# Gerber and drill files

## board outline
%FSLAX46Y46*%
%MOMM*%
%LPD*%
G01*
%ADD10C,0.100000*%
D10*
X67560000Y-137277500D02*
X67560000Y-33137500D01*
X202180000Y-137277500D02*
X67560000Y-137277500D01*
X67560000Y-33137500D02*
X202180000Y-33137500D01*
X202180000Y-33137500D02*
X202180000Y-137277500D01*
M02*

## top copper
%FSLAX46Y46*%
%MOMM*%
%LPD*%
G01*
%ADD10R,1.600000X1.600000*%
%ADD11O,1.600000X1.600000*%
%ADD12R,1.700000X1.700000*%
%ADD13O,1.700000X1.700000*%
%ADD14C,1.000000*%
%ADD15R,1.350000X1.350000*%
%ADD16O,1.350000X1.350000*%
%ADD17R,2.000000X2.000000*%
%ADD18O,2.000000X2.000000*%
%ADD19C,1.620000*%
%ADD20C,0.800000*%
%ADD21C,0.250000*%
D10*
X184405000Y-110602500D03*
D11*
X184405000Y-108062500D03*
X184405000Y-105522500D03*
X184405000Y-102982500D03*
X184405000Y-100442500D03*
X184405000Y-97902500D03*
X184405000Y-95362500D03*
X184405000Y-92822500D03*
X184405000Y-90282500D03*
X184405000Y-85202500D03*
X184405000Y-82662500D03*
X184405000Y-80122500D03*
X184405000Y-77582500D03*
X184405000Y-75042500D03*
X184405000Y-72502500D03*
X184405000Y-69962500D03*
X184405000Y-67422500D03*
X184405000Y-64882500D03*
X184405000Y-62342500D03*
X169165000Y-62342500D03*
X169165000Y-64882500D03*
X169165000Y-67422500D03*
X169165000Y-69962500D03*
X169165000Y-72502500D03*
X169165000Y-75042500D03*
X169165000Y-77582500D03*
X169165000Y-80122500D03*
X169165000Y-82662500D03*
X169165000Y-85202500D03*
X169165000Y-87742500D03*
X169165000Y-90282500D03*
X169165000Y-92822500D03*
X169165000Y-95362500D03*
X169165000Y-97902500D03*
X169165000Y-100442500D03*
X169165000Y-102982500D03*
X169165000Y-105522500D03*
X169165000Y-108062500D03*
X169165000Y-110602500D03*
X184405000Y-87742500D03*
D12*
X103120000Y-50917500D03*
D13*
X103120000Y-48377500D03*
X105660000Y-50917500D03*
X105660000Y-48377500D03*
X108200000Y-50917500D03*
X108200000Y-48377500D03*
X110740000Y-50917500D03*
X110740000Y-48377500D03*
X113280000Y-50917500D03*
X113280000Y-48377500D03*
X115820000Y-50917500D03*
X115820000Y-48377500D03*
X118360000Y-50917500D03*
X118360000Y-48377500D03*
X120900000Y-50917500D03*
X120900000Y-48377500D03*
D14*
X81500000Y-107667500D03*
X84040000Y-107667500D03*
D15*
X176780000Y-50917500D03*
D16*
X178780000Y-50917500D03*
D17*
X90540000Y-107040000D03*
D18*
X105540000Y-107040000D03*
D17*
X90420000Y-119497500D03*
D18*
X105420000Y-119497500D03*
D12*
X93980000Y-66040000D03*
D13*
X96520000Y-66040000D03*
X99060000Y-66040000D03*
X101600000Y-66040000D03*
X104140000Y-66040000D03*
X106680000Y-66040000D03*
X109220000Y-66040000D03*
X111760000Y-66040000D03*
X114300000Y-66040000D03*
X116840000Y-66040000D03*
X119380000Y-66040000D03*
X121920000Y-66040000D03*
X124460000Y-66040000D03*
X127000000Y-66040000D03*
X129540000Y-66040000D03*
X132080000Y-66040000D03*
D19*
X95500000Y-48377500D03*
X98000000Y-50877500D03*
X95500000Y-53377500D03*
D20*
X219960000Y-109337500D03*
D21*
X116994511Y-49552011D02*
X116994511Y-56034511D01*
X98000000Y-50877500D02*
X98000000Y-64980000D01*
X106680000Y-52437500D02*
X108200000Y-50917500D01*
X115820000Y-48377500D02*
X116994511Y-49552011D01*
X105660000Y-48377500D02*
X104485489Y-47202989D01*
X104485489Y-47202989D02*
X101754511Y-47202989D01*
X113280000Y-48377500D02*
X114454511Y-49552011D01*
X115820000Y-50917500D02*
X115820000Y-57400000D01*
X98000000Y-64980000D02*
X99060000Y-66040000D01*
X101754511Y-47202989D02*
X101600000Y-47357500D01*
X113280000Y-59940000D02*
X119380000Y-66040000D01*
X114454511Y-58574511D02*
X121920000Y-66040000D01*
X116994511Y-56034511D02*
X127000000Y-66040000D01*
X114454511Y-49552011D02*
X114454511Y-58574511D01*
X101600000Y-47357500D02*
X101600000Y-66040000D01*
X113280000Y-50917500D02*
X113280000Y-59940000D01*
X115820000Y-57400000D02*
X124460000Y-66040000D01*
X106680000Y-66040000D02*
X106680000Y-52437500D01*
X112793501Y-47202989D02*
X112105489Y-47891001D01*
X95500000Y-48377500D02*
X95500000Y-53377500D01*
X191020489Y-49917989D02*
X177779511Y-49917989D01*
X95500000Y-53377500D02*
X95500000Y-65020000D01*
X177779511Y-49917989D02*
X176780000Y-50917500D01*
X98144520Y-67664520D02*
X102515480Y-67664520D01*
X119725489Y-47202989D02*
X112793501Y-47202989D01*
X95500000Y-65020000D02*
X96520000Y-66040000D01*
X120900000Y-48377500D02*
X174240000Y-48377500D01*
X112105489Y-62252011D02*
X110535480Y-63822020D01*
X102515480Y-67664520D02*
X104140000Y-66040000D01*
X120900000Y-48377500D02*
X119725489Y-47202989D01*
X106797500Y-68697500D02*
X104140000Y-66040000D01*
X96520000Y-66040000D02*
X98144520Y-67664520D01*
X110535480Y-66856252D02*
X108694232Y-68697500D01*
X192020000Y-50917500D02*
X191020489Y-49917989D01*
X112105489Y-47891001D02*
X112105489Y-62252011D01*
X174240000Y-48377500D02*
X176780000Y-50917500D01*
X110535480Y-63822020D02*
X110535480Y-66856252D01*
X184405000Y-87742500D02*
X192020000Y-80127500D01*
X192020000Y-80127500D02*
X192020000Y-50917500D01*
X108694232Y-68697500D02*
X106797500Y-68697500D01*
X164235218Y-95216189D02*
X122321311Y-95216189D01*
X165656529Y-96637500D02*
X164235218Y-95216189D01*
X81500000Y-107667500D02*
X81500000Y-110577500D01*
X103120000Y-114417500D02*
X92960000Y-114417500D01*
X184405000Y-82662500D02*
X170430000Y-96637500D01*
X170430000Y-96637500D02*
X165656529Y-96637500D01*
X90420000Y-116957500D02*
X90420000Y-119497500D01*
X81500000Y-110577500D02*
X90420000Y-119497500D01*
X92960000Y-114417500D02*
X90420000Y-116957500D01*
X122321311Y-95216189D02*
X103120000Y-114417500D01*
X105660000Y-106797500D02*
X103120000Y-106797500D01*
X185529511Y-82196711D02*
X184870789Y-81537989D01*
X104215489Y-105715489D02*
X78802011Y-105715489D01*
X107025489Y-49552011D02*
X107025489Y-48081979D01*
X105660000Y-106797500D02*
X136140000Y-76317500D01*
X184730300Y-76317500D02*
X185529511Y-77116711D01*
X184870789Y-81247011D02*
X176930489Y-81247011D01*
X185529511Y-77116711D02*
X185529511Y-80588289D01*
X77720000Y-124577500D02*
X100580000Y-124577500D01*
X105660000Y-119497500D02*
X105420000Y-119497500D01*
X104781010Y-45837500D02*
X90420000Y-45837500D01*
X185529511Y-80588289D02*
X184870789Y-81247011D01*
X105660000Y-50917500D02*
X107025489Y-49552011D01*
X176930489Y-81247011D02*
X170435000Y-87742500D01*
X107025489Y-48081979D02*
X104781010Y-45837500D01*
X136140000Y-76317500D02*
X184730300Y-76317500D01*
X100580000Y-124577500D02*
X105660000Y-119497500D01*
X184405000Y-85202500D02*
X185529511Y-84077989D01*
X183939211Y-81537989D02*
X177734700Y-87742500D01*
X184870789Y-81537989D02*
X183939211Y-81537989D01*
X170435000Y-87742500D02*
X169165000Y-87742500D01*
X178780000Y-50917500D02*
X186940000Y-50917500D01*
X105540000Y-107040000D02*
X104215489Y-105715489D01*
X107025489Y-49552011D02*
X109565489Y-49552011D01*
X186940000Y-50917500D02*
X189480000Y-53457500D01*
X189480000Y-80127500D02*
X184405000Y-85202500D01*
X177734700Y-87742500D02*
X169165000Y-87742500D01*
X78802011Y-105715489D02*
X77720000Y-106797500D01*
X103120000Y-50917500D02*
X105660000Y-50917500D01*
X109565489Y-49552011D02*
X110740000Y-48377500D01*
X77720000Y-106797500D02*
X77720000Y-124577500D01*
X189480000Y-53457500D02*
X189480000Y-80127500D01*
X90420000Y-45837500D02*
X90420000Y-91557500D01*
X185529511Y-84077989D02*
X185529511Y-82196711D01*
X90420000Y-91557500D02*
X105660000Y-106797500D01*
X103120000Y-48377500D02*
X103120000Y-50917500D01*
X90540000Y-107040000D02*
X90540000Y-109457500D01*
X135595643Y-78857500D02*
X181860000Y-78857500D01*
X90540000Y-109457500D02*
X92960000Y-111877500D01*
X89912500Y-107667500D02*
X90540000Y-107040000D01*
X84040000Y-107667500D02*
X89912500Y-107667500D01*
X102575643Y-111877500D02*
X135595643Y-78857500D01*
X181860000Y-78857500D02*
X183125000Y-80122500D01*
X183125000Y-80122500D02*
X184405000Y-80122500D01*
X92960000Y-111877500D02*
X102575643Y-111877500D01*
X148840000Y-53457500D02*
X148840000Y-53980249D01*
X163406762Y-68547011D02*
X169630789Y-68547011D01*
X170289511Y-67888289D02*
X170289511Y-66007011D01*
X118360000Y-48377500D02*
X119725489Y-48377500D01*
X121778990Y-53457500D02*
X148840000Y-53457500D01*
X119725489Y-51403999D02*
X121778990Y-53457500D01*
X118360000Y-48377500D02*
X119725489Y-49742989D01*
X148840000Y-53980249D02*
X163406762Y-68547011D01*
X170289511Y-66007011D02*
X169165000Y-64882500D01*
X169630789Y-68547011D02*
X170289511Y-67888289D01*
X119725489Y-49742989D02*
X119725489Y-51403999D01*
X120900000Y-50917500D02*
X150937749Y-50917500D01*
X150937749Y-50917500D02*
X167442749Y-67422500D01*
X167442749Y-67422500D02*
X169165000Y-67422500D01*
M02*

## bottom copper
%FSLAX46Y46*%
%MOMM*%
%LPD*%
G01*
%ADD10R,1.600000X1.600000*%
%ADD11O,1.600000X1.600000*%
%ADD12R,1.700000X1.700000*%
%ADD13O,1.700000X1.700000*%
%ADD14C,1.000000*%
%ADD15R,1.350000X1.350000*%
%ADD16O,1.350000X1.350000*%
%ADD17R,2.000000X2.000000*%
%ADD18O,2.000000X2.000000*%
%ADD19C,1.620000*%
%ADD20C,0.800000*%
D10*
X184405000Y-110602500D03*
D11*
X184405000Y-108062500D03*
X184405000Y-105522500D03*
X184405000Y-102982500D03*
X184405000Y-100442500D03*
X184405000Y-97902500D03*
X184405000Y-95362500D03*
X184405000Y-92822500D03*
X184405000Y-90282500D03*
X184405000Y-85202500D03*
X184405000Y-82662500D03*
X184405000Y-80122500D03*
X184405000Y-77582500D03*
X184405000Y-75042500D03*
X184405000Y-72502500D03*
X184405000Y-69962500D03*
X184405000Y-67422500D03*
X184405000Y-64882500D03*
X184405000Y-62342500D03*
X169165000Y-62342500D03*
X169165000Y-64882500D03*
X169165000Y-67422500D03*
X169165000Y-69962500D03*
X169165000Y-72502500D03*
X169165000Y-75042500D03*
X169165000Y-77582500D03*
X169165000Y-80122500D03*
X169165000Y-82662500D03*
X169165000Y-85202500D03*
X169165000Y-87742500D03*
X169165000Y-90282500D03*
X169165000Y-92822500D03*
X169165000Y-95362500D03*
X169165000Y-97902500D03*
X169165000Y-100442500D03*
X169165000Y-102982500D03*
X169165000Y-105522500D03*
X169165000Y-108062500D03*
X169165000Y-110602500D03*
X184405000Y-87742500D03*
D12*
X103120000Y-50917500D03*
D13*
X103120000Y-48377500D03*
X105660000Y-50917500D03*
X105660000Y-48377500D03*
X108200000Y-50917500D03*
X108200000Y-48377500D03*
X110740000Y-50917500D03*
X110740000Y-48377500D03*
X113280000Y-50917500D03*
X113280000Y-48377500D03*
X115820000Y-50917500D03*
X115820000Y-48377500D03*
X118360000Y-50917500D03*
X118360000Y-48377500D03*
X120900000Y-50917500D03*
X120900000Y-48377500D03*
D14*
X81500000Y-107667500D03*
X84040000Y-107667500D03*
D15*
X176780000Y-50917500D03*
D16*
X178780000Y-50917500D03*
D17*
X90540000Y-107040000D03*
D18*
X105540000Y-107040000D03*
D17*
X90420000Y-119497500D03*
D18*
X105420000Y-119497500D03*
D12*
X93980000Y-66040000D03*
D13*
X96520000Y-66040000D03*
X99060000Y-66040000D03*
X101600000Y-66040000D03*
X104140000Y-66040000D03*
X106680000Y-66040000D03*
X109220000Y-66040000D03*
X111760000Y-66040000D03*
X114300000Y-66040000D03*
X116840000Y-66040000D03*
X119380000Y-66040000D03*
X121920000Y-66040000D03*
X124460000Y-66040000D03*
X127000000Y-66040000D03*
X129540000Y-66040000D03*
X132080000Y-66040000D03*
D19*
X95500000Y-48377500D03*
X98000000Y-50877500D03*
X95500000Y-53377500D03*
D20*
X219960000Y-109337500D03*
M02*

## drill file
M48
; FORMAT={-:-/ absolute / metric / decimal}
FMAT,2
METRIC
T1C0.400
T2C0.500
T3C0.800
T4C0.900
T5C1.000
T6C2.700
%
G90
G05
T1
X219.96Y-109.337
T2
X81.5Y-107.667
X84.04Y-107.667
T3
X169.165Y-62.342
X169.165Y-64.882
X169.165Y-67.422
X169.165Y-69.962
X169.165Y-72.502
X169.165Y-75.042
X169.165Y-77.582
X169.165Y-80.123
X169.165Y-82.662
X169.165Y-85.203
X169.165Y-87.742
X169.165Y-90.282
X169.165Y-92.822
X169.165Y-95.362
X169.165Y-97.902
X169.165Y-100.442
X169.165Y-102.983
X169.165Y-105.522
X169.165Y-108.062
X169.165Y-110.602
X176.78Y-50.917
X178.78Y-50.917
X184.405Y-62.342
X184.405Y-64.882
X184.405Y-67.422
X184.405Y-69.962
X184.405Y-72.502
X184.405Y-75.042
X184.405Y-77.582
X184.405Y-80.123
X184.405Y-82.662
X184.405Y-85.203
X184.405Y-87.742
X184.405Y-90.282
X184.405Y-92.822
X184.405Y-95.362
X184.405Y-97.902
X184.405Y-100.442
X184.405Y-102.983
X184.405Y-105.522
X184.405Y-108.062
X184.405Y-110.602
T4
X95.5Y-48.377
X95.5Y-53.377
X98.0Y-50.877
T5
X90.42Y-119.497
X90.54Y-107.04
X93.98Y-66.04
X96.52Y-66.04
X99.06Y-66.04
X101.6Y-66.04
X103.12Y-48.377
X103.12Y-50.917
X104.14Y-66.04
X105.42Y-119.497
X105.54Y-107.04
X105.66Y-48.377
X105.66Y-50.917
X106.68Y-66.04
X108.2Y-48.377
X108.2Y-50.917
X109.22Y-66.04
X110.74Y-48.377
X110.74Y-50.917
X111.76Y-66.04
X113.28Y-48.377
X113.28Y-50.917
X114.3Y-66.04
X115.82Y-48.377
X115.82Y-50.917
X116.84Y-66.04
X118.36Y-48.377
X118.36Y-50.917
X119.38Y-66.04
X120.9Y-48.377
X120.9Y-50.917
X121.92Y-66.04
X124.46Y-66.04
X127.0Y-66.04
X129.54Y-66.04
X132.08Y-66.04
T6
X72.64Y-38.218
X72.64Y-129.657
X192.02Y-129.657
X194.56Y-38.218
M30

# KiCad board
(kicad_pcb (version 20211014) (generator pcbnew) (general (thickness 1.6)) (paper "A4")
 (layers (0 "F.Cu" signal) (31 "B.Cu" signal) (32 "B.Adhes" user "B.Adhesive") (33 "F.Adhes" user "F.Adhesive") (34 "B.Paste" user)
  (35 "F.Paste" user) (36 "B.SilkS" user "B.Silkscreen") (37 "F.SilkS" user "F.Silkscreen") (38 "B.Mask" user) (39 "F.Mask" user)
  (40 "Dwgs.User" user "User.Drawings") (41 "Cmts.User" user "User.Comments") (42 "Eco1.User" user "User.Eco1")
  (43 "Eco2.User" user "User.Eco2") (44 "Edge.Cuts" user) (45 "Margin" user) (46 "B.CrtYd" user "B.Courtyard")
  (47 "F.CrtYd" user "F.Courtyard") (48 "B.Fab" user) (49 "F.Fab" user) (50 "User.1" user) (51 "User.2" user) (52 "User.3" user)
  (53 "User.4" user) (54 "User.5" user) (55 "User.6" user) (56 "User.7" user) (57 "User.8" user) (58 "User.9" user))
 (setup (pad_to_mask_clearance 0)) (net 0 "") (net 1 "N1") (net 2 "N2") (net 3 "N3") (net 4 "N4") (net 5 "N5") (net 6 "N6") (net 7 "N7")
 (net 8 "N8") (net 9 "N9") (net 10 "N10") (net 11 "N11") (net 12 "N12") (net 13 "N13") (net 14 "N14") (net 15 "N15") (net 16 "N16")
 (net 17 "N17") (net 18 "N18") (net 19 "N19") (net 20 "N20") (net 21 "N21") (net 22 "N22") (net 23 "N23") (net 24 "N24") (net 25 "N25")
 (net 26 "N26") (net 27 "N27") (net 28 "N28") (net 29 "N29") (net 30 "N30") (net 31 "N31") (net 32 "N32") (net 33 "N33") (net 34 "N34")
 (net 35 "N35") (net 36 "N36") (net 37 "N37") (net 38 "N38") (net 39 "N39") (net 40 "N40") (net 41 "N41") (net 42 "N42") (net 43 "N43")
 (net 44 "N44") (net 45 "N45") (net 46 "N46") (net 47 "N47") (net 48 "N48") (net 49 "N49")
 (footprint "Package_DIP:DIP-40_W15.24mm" (layer "F.Cu") (at 184.405 110.6025 180)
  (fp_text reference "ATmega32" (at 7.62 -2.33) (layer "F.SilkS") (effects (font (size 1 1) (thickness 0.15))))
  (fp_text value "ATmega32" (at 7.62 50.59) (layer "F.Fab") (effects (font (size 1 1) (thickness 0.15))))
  (pad "1" thru_hole rect (at 0 0 180) (size 1.6 1.6) (drill 0.8) (layers *.Cu *.Mask) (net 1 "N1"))
  (pad "2" thru_hole oval (at 0 2.54 180) (size 1.6 1.6) (drill 0.8) (layers *.Cu *.Mask) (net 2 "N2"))
  (pad "3" thru_hole oval (at 0 5.08 180) (size 1.6 1.6) (drill 0.8) (layers *.Cu *.Mask) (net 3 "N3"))
  (pad "4" thru_hole oval (at 0 7.62 180) (size 1.6 1.6) (drill 0.8) (layers *.Cu *.Mask) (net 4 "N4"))
  (pad "5" thru_hole oval (at 0 10.16 180) (size 1.6 1.6) (drill 0.8) (layers *.Cu *.Mask) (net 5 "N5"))
  (pad "6" thru_hole oval (at 0 12.7 180) (size 1.6 1.6) (drill 0.8) (layers *.Cu *.Mask) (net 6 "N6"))
  (pad "7" thru_hole oval (at 0 15.24 180) (size 1.6 1.6) (drill 0.8) (layers *.Cu *.Mask) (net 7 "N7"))
  (pad "8" thru_hole oval (at 0 17.78 180) (size 1.6 1.6) (drill 0.8) (layers *.Cu *.Mask) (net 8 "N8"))
  (pad "9" thru_hole oval (at 0 20.32 180) (size 1.6 1.6) (drill 0.8) (layers *.Cu *.Mask) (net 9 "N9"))
  (pad "11" thru_hole oval (at 0 25.4 180) (size 1.6 1.6) (drill 0.8) (layers *.Cu *.Mask) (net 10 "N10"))
  (pad "12" thru_hole oval (at 0 27.94 180) (size 1.6 1.6) (drill 0.8) (layers *.Cu *.Mask) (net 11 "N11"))
  (pad "13" thru_hole oval (at 0 30.48 180) (size 1.6 1.6) (drill 0.8) (layers *.Cu *.Mask) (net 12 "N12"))
  (pad "14" thru_hole oval (at 0 33.02 180) (size 1.6 1.6) (drill 0.8) (layers *.Cu *.Mask) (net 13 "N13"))
  (pad "15" thru_hole oval (at 0 35.56 180) (size 1.6 1.6) (drill 0.8) (layers *.Cu *.Mask) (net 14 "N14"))
  (pad "16" thru_hole oval (at 0 38.1 180) (size 1.6 1.6) (drill 0.8) (layers *.Cu *.Mask) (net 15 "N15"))
  (pad "17" thru_hole oval (at 0 40.64 180) (size 1.6 1.6) (drill 0.8) (layers *.Cu *.Mask) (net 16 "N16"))
  (pad "18" thru_hole oval (at 0 43.18 180) (size 1.6 1.6) (drill 0.8) (layers *.Cu *.Mask) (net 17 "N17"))
  (pad "19" thru_hole oval (at 0 45.72 180) (size 1.6 1.6) (drill 0.8) (layers *.Cu *.Mask) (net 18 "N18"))
  (pad "20" thru_hole oval (at 0 48.26 180) (size 1.6 1.6) (drill 0.8) (layers *.Cu *.Mask) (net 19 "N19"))
  (pad "21" thru_hole oval (at 15.24 48.26 180) (size 1.6 1.6) (drill 0.8) (layers *.Cu *.Mask) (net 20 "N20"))
  (pad "22" thru_hole oval (at 15.24 45.72 180) (size 1.6 1.6) (drill 0.8) (layers *.Cu *.Mask))
  (pad "23" thru_hole oval (at 15.24 43.18 180) (size 1.6 1.6) (drill 0.8) (layers *.Cu *.Mask) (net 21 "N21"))
  (pad "24" thru_hole oval (at 15.24 40.64 180) (size 1.6 1.6) (drill 0.8) (layers *.Cu *.Mask) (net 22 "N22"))
  (pad "25" thru_hole oval (at 15.24 38.1 180) (size 1.6 1.6) (drill 0.8) (layers *.Cu *.Mask) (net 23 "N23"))
  (pad "26" thru_hole oval (at 15.24 35.56 180) (size 1.6 1.6) (drill 0.8) (layers *.Cu *.Mask) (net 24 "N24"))
  (pad "27" thru_hole oval (at 15.24 33.02 180) (size 1.6 1.6) (drill 0.8) (layers *.Cu *.Mask) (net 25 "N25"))
  (pad "28" thru_hole oval (at 15.24 30.48 180) (size 1.6 1.6) (drill 0.8) (layers *.Cu *.Mask) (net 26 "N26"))
  (pad "29" thru_hole oval (at 15.24 27.94 180) (size 1.6 1.6) (drill 0.8) (layers *.Cu *.Mask) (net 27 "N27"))
  (pad "30" thru_hole oval (at 15.24 25.4 180) (size 1.6 1.6) (drill 0.8) (layers *.Cu *.Mask) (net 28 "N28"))
  (pad "31" thru_hole oval (at 15.24 22.86 180) (size 1.6 1.6) (drill 0.8) (layers *.Cu *.Mask) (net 10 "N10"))
  (pad "32" thru_hole oval (at 15.24 20.32 180) (size 1.6 1.6) (drill 0.8) (layers *.Cu *.Mask) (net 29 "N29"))
  (pad "33" thru_hole oval (at 15.24 17.78 180) (size 1.6 1.6) (drill 0.8) (layers *.Cu *.Mask) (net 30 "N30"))
  (pad "34" thru_hole oval (at 15.24 15.24 180) (size 1.6 1.6) (drill 0.8) (layers *.Cu *.Mask) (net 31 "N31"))
  (pad "35" thru_hole oval (at 15.24 12.7 180) (size 1.6 1.6) (drill 0.8) (layers *.Cu *.Mask) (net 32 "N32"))
  (pad "36" thru_hole oval (at 15.24 10.16 180) (size 1.6 1.6) (drill 0.8) (layers *.Cu *.Mask) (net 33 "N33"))
  (pad "37" thru_hole oval (at 15.24 7.62 180) (size 1.6 1.6) (drill 0.8) (layers *.Cu *.Mask) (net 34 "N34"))
  (pad "38" thru_hole oval (at 15.24 5.08 180) (size 1.6 1.6) (drill 0.8) (layers *.Cu *.Mask) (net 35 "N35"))
  (pad "39" thru_hole oval (at 15.24 2.54 180) (size 1.6 1.6) (drill 0.8) (layers *.Cu *.Mask) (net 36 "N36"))
  (pad "40" thru_hole oval (at 15.24 0 180) (size 1.6 1.6) (drill 0.8) (layers *.Cu *.Mask) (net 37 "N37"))
  (pad "PIN 10" thru_hole oval (at 0 22.86 180) (size 1.6 1.6) (drill 0.8) (layers *.Cu *.Mask) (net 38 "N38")))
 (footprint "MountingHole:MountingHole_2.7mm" (layer "F.Cu") (at 192.02 129.6575)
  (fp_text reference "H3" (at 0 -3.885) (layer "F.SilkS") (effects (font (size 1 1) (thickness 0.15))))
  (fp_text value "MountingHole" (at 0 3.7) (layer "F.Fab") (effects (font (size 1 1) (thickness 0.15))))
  (pad "" np_thru_hole circle (at 0 0) (size 2.7 2.7) (drill 2.7) (layers *.Cu *.Mask)))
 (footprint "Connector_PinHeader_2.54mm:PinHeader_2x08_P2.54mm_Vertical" (layer "F.Cu") (at 103.12 50.9175 90)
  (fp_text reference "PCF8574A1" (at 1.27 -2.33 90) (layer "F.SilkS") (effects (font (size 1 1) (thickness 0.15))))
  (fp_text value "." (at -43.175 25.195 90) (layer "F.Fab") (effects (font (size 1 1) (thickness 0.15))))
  (pad "1" thru_hole rect (at 0 0 90) (size 1.7 1.7) (drill 1) (layers *.Cu *.Mask) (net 10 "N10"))
  (pad "2" thru_hole oval (at 2.54 0 90) (size 1.7 1.7) (drill 1) (layers *.Cu *.Mask) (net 10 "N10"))
  (pad "3" thru_hole oval (at 0 2.54 90) (size 1.7 1.7) (drill 1) (layers *.Cu *.Mask) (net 10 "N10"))
  (pad "4" thru_hole oval (at 2.54 2.54 90) (size 1.7 1.7) (drill 1) (layers *.Cu *.Mask))
  (pad "5" thru_hole oval (at 0 5.08 90) (size 1.7 1.7) (drill 1) (layers *.Cu *.Mask))
  (pad "6" thru_hole oval (at 2.54 5.08 90) (size 1.7 1.7) (drill 1) (layers *.Cu *.Mask) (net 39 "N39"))
  (pad "7" thru_hole oval (at 0 7.62 90) (size 1.7 1.7) (drill 1) (layers *.Cu *.Mask) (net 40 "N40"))
  (pad "8" thru_hole oval (at 2.54 7.62 90) (size 1.7 1.7) (drill 1) (layers *.Cu *.Mask) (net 10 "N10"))
  (pad "9" thru_hole oval (at 0 10.16 90) (size 1.7 1.7) (drill 1) (layers *.Cu *.Mask))
  (pad "10" thru_hole oval (at 2.54 10.16 90) (size 1.7 1.7) (drill 1) (layers *.Cu *.Mask))
  (pad "11" thru_hole oval (at 0 12.7 90) (size 1.7 1.7) (drill 1) (layers *.Cu *.Mask))
  (pad "12" thru_hole oval (at 2.54 12.7 90) (size 1.7 1.7) (drill 1) (layers *.Cu *.Mask))
  (pad "13" thru_hole oval (at 0 15.24 90) (size 1.7 1.7) (drill 1) (layers *.Cu *.Mask) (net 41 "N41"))
  (pad "14" thru_hole oval (at 2.54 15.24 90) (size 1.7 1.7) (drill 1) (layers *.Cu *.Mask) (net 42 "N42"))
  (pad "15" thru_hole oval (at 0 17.78 90) (size 1.7 1.7) (drill 1) (layers *.Cu *.Mask) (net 21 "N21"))
  (pad "16" thru_hole oval (at 2.54 17.78 90) (size 1.7 1.7) (drill 1) (layers *.Cu *.Mask) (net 38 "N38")))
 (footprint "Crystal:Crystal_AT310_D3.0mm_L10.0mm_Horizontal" (layer "F.Cu") (at 81.5 107.6675)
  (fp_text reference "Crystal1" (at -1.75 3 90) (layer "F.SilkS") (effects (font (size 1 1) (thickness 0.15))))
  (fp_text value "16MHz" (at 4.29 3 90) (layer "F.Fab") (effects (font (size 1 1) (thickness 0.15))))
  (pad "1" thru_hole circle (at 0 0) (size 1 1) (drill 0.5) (layers *.Cu *.Mask) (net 11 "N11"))
  (pad "2" thru_hole circle (at 2.54 0) (size 1 1) (drill 0.5) (layers *.Cu *.Mask) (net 12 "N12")))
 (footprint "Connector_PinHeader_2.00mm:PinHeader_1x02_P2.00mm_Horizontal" (layer "F.Cu") (at 176.78 50.9175 90)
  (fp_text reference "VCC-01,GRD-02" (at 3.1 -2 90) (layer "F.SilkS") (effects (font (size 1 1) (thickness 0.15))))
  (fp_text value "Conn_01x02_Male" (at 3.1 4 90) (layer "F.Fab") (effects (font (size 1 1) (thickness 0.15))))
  (pad "1" thru_hole rect (at 0 0 90) (size 1.35 1.35) (drill 0.8) (layers *.Cu *.Mask) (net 38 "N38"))
  (pad "2" thru_hole oval (at 0 2 90) (size 1.35 1.35) (drill 0.8) (layers *.Cu *.Mask) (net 10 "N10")))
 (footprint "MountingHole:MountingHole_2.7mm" (layer "F.Cu") (at 72.64 129.6575)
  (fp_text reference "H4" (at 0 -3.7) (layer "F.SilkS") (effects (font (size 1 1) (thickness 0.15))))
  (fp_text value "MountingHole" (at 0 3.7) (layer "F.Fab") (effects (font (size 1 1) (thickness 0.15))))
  (pad "" np_thru_hole circle (at 0 0) (size 2.7 2.7) (drill 2.7) (layers *.Cu *.Mask)))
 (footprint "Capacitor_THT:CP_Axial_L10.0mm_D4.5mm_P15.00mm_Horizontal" (layer "F.Cu") (at 90.54 107.04)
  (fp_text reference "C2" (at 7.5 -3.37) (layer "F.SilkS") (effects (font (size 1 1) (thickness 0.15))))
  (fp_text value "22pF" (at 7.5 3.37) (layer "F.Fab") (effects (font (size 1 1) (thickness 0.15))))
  (pad "1" thru_hole rect (at 0 0) (size 2 2) (drill 1) (layers *.Cu *.Mask) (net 12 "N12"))
  (pad "2" thru_hole oval (at 15 0) (size 2 2) (drill 1) (layers *.Cu *.Mask) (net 10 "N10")))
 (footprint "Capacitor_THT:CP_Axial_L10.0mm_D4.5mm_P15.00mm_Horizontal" (layer "F.Cu") (at 90.42 119.4975)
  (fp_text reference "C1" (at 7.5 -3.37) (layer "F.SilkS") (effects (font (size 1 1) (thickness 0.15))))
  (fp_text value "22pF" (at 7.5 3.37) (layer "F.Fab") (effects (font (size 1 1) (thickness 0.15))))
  (pad "1" thru_hole rect (at 0 0) (size 2 2) (drill 1) (layers *.Cu *.Mask) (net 11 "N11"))
  (pad "2" thru_hole oval (at 15 0) (size 2 2) (drill 1) (layers *.Cu *.Mask) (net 10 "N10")))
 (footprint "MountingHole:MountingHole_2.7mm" (layer "F.Cu") (at 194.56 38.2175)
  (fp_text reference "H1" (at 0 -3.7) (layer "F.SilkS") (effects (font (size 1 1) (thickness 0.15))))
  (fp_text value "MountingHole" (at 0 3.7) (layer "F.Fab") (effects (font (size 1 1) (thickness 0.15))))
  (pad "" np_thru_hole circle (at 0 0) (size 2.7 2.7) (drill 2.7) (layers *.Cu *.Mask)))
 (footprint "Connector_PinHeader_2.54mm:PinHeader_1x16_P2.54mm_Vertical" (layer "F.Cu") (at 93.98 66.04 90)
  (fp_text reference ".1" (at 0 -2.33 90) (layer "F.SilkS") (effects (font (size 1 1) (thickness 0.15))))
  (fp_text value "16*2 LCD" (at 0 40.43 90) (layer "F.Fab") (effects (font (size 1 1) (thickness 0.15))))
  (pad "1" thru_hole rect (at 0 0 90) (size 1.7 1.7) (drill 1) (layers *.Cu *.Mask) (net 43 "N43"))
  (pad "2" thru_hole oval (at 0 2.54 90) (size 1.7 1.7) (drill 1) (layers *.Cu *.Mask) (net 38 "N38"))
  (pad "3" thru_hole oval (at 0 5.08 90) (size 1.7 1.7) (drill 1) (layers *.Cu *.Mask))
  (pad "4" thru_hole oval (at 0 7.62 90) (size 1.7 1.7) (drill 1) (layers *.Cu *.Mask))
  (pad "5" thru_hole oval (at 0 10.16 90) (size 1.7 1.7) (drill 1) (layers *.Cu *.Mask) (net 38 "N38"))
  (pad "6" thru_hole oval (at 0 12.7 90) (size 1.7 1.7) (drill 1) (layers *.Cu *.Mask))
  (pad "7" thru_hole oval (at 0 15.24 90) (size 1.7 1.7) (drill 1) (layers *.Cu *.Mask) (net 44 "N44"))
  (pad "8" thru_hole oval (at 0 17.78 90) (size 1.7 1.7) (drill 1) (layers *.Cu *.Mask) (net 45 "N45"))
  (pad "9" thru_hole oval (at 0 20.32 90) (size 1.7 1.7) (drill 1) (layers *.Cu *.Mask) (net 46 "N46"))
  (pad "10" thru_hole oval (at 0 22.86 90) (size 1.7 1.7) (drill 1) (layers *.Cu *.Mask) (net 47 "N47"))
  (pad "11" thru_hole oval (at 0 25.4 90) (size 1.7 1.7) (drill 1) (layers *.Cu *.Mask))
  (pad "12" thru_hole oval (at 0 27.94 90) (size 1.7 1.7) (drill 1) (layers *.Cu *.Mask))
  (pad "13" thru_hole oval (at 0 30.48 90) (size 1.7 1.7) (drill 1) (layers *.Cu *.Mask))
  (pad "14" thru_hole oval (at 0 33.02 90) (size 1.7 1.7) (drill 1) (layers *.Cu *.Mask))
  (pad "15" thru_hole oval (at 0 35.56 90) (size 1.7 1.7) (drill 1) (layers *.Cu *.Mask) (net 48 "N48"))
  (pad "16" thru_hole oval (at 0 38.1 90) (size 1.7 1.7) (drill 1) (layers *.Cu *.Mask) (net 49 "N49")))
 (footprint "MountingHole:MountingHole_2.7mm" (layer "F.Cu") (at 72.64 38.2175)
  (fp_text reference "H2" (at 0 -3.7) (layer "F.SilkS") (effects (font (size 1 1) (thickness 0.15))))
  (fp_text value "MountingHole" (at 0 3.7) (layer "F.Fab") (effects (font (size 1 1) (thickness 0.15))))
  (pad "" np_thru_hole circle (at 0 0) (size 2.7 2.7) (drill 2.7) (layers *.Cu *.Mask)))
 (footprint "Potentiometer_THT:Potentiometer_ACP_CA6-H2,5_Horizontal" (layer "F.Cu") (at 95.5 48.3775)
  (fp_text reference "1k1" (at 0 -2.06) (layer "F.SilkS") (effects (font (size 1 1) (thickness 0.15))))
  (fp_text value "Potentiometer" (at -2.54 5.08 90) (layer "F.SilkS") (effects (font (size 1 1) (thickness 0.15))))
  (pad "1" thru_hole circle (at 0 0) (size 1.62 1.62) (drill 0.9) (layers *.Cu *.Mask) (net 38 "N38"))
  (pad "2" thru_hole circle (at 2.5 2.5) (size 1.62 1.62) (drill 0.9) (layers *.Cu *.Mask))
  (pad "3" thru_hole circle (at 0 5) (size 1.62 1.62) (drill 0.9) (layers *.Cu *.Mask) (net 38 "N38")))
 (gr_line (start 67.56 137.2775) (end 67.56 33.1375) (layer "Edge.Cuts") (width 0.1))
 (gr_line (start 202.18 137.2775) (end 67.56 137.2775) (layer "Edge.Cuts") (width 0.1))
 (gr_line (start 67.56 33.1375) (end 202.18 33.1375) (layer "Edge.Cuts") (width 0.1))
 (gr_line (start 202.18 33.1375) (end 202.18 137.2775) (layer "Edge.Cuts") (width 0.1))
 (segment (start 116.994511 49.552011) (end 116.994511 56.034511) (width 0.25) (layer "F.Cu") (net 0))
 (segment (start 98 50.8775) (end 98 64.98) (width 0.25) (layer "F.Cu") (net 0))
 (segment (start 106.68 52.4375) (end 108.2 50.9175) (width 0.25) (layer "F.Cu") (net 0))
 (segment (start 115.82 48.3775) (end 116.994511 49.552011) (width 0.25) (layer "F.Cu") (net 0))
 (segment (start 105.66 48.3775) (end 104.485489 47.202989) (width 0.25) (layer "F.Cu") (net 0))
 (segment (start 104.485489 47.202989) (end 101.754511 47.202989) (width 0.25) (layer "F.Cu") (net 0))
 (segment (start 113.28 48.3775) (end 114.454511 49.552011) (width 0.25) (layer "F.Cu") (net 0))
 (segment (start 115.82 50.9175) (end 115.82 57.4) (width 0.25) (layer "F.Cu") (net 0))
 (segment (start 98 64.98) (end 99.06 66.04) (width 0.25) (layer "F.Cu") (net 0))
 (segment (start 101.754511 47.202989) (end 101.6 47.3575) (width 0.25) (layer "F.Cu") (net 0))
 (segment (start 113.28 59.94) (end 119.38 66.04) (width 0.25) (layer "F.Cu") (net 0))
 (segment (start 114.454511 58.574511) (end 121.92 66.04) (width 0.25) (layer "F.Cu") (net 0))
 (segment (start 116.994511 56.034511) (end 127 66.04) (width 0.25) (layer "F.Cu") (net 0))
 (segment (start 114.454511 49.552011) (end 114.454511 58.574511) (width 0.25) (layer "F.Cu") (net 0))
 (segment (start 101.6 47.3575) (end 101.6 66.04) (width 0.25) (layer "F.Cu") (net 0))
 (segment (start 113.28 50.9175) (end 113.28 59.94) (width 0.25) (layer "F.Cu") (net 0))
 (segment (start 115.82 57.4) (end 124.46 66.04) (width 0.25) (layer "F.Cu") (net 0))
 (segment (start 106.68 66.04) (end 106.68 52.4375) (width 0.25) (layer "F.Cu") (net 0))
 (via (at 219.96 109.3375) (size 0.8) (drill 0.4) (layers "F.Cu" "B.Cu") (free) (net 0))
 (segment (start 112.793501 47.202989) (end 112.105489 47.891001) (width 0.25) (layer "F.Cu") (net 38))
 (segment (start 95.5 48.3775) (end 95.5 53.3775) (width 0.25) (layer "F.Cu") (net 38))
 (segment (start 191.020489 49.917989) (end 177.779511 49.917989) (width 0.25) (layer "F.Cu") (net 38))
 (segment (start 95.5 53.3775) (end 95.5 65.02) (width 0.25) (layer "F.Cu") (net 38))
 (segment (start 177.779511 49.917989) (end 176.78 50.9175) (width 0.25) (layer "F.Cu") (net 38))
 (segment (start 98.14452 67.66452) (end 102.51548 67.66452) (width 0.25) (layer "F.Cu") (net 38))
 (segment (start 119.725489 47.202989) (end 112.793501 47.202989) (width 0.25) (layer "F.Cu") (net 38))
 (segment (start 95.5 65.02) (end 96.52 66.04) (width 0.25) (layer "F.Cu") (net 38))
 (segment (start 120.9 48.3775) (end 174.24 48.3775) (width 0.25) (layer "F.Cu") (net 38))
 (segment (start 112.105489 62.252011) (end 110.53548 63.82202) (width 0.25) (layer "F.Cu") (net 38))
 (segment (start 102.51548 67.66452) (end 104.14 66.04) (width 0.25) (layer "F.Cu") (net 38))
 (segment (start 120.9 48.3775) (end 119.725489 47.202989) (width 0.25) (layer "F.Cu") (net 38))
 (segment (start 106.7975 68.6975) (end 104.14 66.04) (width 0.25) (layer "F.Cu") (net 38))
 (segment (start 96.52 66.04) (end 98.14452 67.66452) (width 0.25) (layer "F.Cu") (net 38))
 (segment (start 110.53548 66.856252) (end 108.694232 68.6975) (width 0.25) (layer "F.Cu") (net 38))
 (segment (start 192.02 50.9175) (end 191.020489 49.917989) (width 0.25) (layer "F.Cu") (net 38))
 (segment (start 112.105489 47.891001) (end 112.105489 62.252011) (width 0.25) (layer "F.Cu") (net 38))
 (segment (start 174.24 48.3775) (end 176.78 50.9175) (width 0.25) (layer "F.Cu") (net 38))
 (segment (start 110.53548 63.82202) (end 110.53548 66.856252) (width 0.25) (layer "F.Cu") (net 38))
 (segment (start 184.405 87.7425) (end 192.02 80.1275) (width 0.25) (layer "F.Cu") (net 38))
 (segment (start 192.02 80.1275) (end 192.02 50.9175) (width 0.25) (layer "F.Cu") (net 38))
 (segment (start 108.694232 68.6975) (end 106.7975 68.6975) (width 0.25) (layer "F.Cu") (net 38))
 (segment (start 164.235218 95.216189) (end 122.321311 95.216189) (width 0.25) (layer "F.Cu") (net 11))
 (segment (start 165.656529 96.6375) (end 164.235218 95.216189) (width 0.25) (layer "F.Cu") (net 11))
 (segment (start 81.5 107.6675) (end 81.5 110.5775) (width 0.25) (layer "F.Cu") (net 11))
 (segment (start 103.12 114.4175) (end 92.96 114.4175) (width 0.25) (layer "F.Cu") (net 11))
 (segment (start 184.405 82.6625) (end 170.43 96.6375) (width 0.25) (layer "F.Cu") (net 11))
 (segment (start 170.43 96.6375) (end 165.656529 96.6375) (width 0.25) (layer "F.Cu") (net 11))
 (segment (start 90.42 116.9575) (end 90.42 119.4975) (width 0.25) (layer "F.Cu") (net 11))
 (segment (start 81.5 110.5775) (end 90.42 119.4975) (width 0.25) (layer "F.Cu") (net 11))
 (segment (start 92.96 114.4175) (end 90.42 116.9575) (width 0.25) (layer "F.Cu") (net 11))
 (segment (start 122.321311 95.216189) (end 103.12 114.4175) (width 0.25) (layer "F.Cu") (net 11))
 (segment (start 105.66 106.7975) (end 103.12 106.7975) (width 0.25) (layer "F.Cu") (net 10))
 (segment (start 185.529511 82.196711) (end 184.870789 81.537989) (width 0.25) (layer "F.Cu") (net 10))
 (segment (start 104.215489 105.715489) (end 78.802011 105.715489) (width 0.25) (layer "F.Cu") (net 10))
 (segment (start 107.025489 49.552011) (end 107.025489 48.081979) (width 0.25) (layer "F.Cu") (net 10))
 (segment (start 105.66 106.7975) (end 136.14 76.3175) (width 0.25) (layer "F.Cu") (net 10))
 (segment (start 184.7303 76.3175) (end 185.529511 77.116711) (width 0.25) (layer "F.Cu") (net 10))
 (segment (start 184.870789 81.247011) (end 176.930489 81.247011) (width 0.25) (layer "F.Cu") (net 10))
 (segment (start 185.529511 77.116711) (end 185.529511 80.588289) (width 0.25) (layer "F.Cu") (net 10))
 (segment (start 77.72 124.5775) (end 100.58 124.5775) (width 0.25) (layer "F.Cu") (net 10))
 (segment (start 105.66 119.4975) (end 105.42 119.4975) (width 0.25) (layer "F.Cu") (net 10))
 (segment (start 104.78101 45.8375) (end 90.42 45.8375) (width 0.25) (layer "F.Cu") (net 10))
 (segment (start 185.529511 80.588289) (end 184.870789 81.247011) (width 0.25) (layer "F.Cu") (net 10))
 (segment (start 105.66 50.9175) (end 107.025489 49.552011) (width 0.25) (layer "F.Cu") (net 10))
 (segment (start 176.930489 81.247011) (end 170.435 87.7425) (width 0.25) (layer "F.Cu") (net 10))
 (segment (start 107.025489 48.081979) (end 104.78101 45.8375) (width 0.25) (layer "F.Cu") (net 10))
 (segment (start 136.14 76.3175) (end 184.7303 76.3175) (width 0.25) (layer "F.Cu") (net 10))
 (segment (start 100.58 124.5775) (end 105.66 119.4975) (width 0.25) (layer "F.Cu") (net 10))
 (segment (start 184.405 85.2025) (end 185.529511 84.077989) (width 0.25) (layer "F.Cu") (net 10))
 (segment (start 183.939211 81.537989) (end 177.7347 87.7425) (width 0.25) (layer "F.Cu") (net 10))
 (segment (start 184.870789 81.537989) (end 183.939211 81.537989) (width 0.25) (layer "F.Cu") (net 10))
 (segment (start 170.435 87.7425) (end 169.165 87.7425) (width 0.25) (layer "F.Cu") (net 10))
 (segment (start 178.78 50.9175) (end 186.94 50.9175) (width 0.25) (layer "F.Cu") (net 10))
 (segment (start 105.54 107.04) (end 104.215489 105.715489) (width 0.25) (layer "F.Cu") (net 10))
 (segment (start 107.025489 49.552011) (end 109.565489 49.552011) (width 0.25) (layer "F.Cu") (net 10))
 (segment (start 186.94 50.9175) (end 189.48 53.4575) (width 0.25) (layer "F.Cu") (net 10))
 (segment (start 189.48 80.1275) (end 184.405 85.2025) (width 0.25) (layer "F.Cu") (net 10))
 (segment (start 177.7347 87.7425) (end 169.165 87.7425) (width 0.25) (layer "F.Cu") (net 10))
 (segment (start 78.802011 105.715489) (end 77.72 106.7975) (width 0.25) (layer "F.Cu") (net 10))
 (segment (start 103.12 50.9175) (end 105.66 50.9175) (width 0.25) (layer "F.Cu") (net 10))
 (segment (start 109.565489 49.552011) (end 110.74 48.3775) (width 0.25) (layer "F.Cu") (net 10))
 (segment (start 77.72 106.7975) (end 77.72 124.5775) (width 0.25) (layer "F.Cu") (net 10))
 (segment (start 189.48 53.4575) (end 189.48 80.1275) (width 0.25) (layer "F.Cu") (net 10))
 (segment (start 90.42 45.8375) (end 90.42 91.5575) (width 0.25) (layer "F.Cu") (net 10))
 (segment (start 185.529511 84.077989) (end 185.529511 82.196711) (width 0.25) (layer "F.Cu") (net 10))
 (segment (start 90.42 91.5575) (end 105.66 106.7975) (width 0.25) (layer "F.Cu") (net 10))
 (segment (start 103.12 48.3775) (end 103.12 50.9175) (width 0.25) (layer "F.Cu") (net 10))
 (segment (start 90.54 107.04) (end 90.54 109.4575) (width 0.25) (layer "F.Cu") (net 12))
 (segment (start 135.595643 78.8575) (end 181.86 78.8575) (width 0.25) (layer "F.Cu") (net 12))
 (segment (start 90.54 109.4575) (end 92.96 111.8775) (width 0.25) (layer "F.Cu") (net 12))
 (segment (start 89.9125 107.6675) (end 90.54 107.04) (width 0.25) (layer "F.Cu") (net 12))
 (segment (start 84.04 107.6675) (end 89.9125 107.6675) (width 0.25) (layer "F.Cu") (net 12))
 (segment (start 102.575643 111.8775) (end 135.595643 78.8575) (width 0.25) (layer "F.Cu") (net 12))
 (segment (start 181.86 78.8575) (end 183.125 80.1225) (width 0.25) (layer "F.Cu") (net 12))
 (segment (start 183.125 80.1225) (end 184.405 80.1225) (width 0.25) (layer "F.Cu") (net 12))
 (segment (start 92.96 111.8775) (end 102.575643 111.8775) (width 0.25) (layer "F.Cu") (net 12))
 (segment (start 148.84 53.4575) (end 148.84 53.980249) (width 0.25) (layer "F.Cu") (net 42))
 (segment (start 163.406762 68.547011) (end 169.630789 68.547011) (width 0.25) (layer "F.Cu") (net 42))
 (segment (start 170.289511 67.888289) (end 170.289511 66.007011) (width 0.25) (layer "F.Cu") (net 42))
 (segment (start 118.36 48.3775) (end 119.725489 48.3775) (width 0.25) (layer "F.Cu") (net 42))
 (segment (start 121.77899 53.4575) (end 148.84 53.4575) (width 0.25) (layer "F.Cu") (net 42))
 (segment (start 119.725489 51.403999) (end 121.77899 53.4575) (width 0.25) (layer "F.Cu") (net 42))
 (segment (start 118.36 48.3775) (end 119.725489 49.742989) (width 0.25) (layer "F.Cu") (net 42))
 (segment (start 148.84 53.980249) (end 163.406762 68.547011) (width 0.25) (layer "F.Cu") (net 42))
 (segment (start 170.289511 66.007011) (end 169.165 64.8825) (width 0.25) (layer "F.Cu") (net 42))
 (segment (start 169.630789 68.547011) (end 170.289511 67.888289) (width 0.25) (layer "F.Cu") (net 42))
 (segment (start 119.725489 49.742989) (end 119.725489 51.403999) (width 0.25) (layer "F.Cu") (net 42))
 (segment (start 120.9 50.9175) (end 150.937749 50.9175) (width 0.25) (layer "F.Cu") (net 21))
 (segment (start 150.937749 50.9175) (end 167.442749 67.4225) (width 0.25) (layer "F.Cu") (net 21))
 (segment (start 167.442749 67.4225) (end 169.165 67.4225) (width 0.25) (layer "F.Cu") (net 21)))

